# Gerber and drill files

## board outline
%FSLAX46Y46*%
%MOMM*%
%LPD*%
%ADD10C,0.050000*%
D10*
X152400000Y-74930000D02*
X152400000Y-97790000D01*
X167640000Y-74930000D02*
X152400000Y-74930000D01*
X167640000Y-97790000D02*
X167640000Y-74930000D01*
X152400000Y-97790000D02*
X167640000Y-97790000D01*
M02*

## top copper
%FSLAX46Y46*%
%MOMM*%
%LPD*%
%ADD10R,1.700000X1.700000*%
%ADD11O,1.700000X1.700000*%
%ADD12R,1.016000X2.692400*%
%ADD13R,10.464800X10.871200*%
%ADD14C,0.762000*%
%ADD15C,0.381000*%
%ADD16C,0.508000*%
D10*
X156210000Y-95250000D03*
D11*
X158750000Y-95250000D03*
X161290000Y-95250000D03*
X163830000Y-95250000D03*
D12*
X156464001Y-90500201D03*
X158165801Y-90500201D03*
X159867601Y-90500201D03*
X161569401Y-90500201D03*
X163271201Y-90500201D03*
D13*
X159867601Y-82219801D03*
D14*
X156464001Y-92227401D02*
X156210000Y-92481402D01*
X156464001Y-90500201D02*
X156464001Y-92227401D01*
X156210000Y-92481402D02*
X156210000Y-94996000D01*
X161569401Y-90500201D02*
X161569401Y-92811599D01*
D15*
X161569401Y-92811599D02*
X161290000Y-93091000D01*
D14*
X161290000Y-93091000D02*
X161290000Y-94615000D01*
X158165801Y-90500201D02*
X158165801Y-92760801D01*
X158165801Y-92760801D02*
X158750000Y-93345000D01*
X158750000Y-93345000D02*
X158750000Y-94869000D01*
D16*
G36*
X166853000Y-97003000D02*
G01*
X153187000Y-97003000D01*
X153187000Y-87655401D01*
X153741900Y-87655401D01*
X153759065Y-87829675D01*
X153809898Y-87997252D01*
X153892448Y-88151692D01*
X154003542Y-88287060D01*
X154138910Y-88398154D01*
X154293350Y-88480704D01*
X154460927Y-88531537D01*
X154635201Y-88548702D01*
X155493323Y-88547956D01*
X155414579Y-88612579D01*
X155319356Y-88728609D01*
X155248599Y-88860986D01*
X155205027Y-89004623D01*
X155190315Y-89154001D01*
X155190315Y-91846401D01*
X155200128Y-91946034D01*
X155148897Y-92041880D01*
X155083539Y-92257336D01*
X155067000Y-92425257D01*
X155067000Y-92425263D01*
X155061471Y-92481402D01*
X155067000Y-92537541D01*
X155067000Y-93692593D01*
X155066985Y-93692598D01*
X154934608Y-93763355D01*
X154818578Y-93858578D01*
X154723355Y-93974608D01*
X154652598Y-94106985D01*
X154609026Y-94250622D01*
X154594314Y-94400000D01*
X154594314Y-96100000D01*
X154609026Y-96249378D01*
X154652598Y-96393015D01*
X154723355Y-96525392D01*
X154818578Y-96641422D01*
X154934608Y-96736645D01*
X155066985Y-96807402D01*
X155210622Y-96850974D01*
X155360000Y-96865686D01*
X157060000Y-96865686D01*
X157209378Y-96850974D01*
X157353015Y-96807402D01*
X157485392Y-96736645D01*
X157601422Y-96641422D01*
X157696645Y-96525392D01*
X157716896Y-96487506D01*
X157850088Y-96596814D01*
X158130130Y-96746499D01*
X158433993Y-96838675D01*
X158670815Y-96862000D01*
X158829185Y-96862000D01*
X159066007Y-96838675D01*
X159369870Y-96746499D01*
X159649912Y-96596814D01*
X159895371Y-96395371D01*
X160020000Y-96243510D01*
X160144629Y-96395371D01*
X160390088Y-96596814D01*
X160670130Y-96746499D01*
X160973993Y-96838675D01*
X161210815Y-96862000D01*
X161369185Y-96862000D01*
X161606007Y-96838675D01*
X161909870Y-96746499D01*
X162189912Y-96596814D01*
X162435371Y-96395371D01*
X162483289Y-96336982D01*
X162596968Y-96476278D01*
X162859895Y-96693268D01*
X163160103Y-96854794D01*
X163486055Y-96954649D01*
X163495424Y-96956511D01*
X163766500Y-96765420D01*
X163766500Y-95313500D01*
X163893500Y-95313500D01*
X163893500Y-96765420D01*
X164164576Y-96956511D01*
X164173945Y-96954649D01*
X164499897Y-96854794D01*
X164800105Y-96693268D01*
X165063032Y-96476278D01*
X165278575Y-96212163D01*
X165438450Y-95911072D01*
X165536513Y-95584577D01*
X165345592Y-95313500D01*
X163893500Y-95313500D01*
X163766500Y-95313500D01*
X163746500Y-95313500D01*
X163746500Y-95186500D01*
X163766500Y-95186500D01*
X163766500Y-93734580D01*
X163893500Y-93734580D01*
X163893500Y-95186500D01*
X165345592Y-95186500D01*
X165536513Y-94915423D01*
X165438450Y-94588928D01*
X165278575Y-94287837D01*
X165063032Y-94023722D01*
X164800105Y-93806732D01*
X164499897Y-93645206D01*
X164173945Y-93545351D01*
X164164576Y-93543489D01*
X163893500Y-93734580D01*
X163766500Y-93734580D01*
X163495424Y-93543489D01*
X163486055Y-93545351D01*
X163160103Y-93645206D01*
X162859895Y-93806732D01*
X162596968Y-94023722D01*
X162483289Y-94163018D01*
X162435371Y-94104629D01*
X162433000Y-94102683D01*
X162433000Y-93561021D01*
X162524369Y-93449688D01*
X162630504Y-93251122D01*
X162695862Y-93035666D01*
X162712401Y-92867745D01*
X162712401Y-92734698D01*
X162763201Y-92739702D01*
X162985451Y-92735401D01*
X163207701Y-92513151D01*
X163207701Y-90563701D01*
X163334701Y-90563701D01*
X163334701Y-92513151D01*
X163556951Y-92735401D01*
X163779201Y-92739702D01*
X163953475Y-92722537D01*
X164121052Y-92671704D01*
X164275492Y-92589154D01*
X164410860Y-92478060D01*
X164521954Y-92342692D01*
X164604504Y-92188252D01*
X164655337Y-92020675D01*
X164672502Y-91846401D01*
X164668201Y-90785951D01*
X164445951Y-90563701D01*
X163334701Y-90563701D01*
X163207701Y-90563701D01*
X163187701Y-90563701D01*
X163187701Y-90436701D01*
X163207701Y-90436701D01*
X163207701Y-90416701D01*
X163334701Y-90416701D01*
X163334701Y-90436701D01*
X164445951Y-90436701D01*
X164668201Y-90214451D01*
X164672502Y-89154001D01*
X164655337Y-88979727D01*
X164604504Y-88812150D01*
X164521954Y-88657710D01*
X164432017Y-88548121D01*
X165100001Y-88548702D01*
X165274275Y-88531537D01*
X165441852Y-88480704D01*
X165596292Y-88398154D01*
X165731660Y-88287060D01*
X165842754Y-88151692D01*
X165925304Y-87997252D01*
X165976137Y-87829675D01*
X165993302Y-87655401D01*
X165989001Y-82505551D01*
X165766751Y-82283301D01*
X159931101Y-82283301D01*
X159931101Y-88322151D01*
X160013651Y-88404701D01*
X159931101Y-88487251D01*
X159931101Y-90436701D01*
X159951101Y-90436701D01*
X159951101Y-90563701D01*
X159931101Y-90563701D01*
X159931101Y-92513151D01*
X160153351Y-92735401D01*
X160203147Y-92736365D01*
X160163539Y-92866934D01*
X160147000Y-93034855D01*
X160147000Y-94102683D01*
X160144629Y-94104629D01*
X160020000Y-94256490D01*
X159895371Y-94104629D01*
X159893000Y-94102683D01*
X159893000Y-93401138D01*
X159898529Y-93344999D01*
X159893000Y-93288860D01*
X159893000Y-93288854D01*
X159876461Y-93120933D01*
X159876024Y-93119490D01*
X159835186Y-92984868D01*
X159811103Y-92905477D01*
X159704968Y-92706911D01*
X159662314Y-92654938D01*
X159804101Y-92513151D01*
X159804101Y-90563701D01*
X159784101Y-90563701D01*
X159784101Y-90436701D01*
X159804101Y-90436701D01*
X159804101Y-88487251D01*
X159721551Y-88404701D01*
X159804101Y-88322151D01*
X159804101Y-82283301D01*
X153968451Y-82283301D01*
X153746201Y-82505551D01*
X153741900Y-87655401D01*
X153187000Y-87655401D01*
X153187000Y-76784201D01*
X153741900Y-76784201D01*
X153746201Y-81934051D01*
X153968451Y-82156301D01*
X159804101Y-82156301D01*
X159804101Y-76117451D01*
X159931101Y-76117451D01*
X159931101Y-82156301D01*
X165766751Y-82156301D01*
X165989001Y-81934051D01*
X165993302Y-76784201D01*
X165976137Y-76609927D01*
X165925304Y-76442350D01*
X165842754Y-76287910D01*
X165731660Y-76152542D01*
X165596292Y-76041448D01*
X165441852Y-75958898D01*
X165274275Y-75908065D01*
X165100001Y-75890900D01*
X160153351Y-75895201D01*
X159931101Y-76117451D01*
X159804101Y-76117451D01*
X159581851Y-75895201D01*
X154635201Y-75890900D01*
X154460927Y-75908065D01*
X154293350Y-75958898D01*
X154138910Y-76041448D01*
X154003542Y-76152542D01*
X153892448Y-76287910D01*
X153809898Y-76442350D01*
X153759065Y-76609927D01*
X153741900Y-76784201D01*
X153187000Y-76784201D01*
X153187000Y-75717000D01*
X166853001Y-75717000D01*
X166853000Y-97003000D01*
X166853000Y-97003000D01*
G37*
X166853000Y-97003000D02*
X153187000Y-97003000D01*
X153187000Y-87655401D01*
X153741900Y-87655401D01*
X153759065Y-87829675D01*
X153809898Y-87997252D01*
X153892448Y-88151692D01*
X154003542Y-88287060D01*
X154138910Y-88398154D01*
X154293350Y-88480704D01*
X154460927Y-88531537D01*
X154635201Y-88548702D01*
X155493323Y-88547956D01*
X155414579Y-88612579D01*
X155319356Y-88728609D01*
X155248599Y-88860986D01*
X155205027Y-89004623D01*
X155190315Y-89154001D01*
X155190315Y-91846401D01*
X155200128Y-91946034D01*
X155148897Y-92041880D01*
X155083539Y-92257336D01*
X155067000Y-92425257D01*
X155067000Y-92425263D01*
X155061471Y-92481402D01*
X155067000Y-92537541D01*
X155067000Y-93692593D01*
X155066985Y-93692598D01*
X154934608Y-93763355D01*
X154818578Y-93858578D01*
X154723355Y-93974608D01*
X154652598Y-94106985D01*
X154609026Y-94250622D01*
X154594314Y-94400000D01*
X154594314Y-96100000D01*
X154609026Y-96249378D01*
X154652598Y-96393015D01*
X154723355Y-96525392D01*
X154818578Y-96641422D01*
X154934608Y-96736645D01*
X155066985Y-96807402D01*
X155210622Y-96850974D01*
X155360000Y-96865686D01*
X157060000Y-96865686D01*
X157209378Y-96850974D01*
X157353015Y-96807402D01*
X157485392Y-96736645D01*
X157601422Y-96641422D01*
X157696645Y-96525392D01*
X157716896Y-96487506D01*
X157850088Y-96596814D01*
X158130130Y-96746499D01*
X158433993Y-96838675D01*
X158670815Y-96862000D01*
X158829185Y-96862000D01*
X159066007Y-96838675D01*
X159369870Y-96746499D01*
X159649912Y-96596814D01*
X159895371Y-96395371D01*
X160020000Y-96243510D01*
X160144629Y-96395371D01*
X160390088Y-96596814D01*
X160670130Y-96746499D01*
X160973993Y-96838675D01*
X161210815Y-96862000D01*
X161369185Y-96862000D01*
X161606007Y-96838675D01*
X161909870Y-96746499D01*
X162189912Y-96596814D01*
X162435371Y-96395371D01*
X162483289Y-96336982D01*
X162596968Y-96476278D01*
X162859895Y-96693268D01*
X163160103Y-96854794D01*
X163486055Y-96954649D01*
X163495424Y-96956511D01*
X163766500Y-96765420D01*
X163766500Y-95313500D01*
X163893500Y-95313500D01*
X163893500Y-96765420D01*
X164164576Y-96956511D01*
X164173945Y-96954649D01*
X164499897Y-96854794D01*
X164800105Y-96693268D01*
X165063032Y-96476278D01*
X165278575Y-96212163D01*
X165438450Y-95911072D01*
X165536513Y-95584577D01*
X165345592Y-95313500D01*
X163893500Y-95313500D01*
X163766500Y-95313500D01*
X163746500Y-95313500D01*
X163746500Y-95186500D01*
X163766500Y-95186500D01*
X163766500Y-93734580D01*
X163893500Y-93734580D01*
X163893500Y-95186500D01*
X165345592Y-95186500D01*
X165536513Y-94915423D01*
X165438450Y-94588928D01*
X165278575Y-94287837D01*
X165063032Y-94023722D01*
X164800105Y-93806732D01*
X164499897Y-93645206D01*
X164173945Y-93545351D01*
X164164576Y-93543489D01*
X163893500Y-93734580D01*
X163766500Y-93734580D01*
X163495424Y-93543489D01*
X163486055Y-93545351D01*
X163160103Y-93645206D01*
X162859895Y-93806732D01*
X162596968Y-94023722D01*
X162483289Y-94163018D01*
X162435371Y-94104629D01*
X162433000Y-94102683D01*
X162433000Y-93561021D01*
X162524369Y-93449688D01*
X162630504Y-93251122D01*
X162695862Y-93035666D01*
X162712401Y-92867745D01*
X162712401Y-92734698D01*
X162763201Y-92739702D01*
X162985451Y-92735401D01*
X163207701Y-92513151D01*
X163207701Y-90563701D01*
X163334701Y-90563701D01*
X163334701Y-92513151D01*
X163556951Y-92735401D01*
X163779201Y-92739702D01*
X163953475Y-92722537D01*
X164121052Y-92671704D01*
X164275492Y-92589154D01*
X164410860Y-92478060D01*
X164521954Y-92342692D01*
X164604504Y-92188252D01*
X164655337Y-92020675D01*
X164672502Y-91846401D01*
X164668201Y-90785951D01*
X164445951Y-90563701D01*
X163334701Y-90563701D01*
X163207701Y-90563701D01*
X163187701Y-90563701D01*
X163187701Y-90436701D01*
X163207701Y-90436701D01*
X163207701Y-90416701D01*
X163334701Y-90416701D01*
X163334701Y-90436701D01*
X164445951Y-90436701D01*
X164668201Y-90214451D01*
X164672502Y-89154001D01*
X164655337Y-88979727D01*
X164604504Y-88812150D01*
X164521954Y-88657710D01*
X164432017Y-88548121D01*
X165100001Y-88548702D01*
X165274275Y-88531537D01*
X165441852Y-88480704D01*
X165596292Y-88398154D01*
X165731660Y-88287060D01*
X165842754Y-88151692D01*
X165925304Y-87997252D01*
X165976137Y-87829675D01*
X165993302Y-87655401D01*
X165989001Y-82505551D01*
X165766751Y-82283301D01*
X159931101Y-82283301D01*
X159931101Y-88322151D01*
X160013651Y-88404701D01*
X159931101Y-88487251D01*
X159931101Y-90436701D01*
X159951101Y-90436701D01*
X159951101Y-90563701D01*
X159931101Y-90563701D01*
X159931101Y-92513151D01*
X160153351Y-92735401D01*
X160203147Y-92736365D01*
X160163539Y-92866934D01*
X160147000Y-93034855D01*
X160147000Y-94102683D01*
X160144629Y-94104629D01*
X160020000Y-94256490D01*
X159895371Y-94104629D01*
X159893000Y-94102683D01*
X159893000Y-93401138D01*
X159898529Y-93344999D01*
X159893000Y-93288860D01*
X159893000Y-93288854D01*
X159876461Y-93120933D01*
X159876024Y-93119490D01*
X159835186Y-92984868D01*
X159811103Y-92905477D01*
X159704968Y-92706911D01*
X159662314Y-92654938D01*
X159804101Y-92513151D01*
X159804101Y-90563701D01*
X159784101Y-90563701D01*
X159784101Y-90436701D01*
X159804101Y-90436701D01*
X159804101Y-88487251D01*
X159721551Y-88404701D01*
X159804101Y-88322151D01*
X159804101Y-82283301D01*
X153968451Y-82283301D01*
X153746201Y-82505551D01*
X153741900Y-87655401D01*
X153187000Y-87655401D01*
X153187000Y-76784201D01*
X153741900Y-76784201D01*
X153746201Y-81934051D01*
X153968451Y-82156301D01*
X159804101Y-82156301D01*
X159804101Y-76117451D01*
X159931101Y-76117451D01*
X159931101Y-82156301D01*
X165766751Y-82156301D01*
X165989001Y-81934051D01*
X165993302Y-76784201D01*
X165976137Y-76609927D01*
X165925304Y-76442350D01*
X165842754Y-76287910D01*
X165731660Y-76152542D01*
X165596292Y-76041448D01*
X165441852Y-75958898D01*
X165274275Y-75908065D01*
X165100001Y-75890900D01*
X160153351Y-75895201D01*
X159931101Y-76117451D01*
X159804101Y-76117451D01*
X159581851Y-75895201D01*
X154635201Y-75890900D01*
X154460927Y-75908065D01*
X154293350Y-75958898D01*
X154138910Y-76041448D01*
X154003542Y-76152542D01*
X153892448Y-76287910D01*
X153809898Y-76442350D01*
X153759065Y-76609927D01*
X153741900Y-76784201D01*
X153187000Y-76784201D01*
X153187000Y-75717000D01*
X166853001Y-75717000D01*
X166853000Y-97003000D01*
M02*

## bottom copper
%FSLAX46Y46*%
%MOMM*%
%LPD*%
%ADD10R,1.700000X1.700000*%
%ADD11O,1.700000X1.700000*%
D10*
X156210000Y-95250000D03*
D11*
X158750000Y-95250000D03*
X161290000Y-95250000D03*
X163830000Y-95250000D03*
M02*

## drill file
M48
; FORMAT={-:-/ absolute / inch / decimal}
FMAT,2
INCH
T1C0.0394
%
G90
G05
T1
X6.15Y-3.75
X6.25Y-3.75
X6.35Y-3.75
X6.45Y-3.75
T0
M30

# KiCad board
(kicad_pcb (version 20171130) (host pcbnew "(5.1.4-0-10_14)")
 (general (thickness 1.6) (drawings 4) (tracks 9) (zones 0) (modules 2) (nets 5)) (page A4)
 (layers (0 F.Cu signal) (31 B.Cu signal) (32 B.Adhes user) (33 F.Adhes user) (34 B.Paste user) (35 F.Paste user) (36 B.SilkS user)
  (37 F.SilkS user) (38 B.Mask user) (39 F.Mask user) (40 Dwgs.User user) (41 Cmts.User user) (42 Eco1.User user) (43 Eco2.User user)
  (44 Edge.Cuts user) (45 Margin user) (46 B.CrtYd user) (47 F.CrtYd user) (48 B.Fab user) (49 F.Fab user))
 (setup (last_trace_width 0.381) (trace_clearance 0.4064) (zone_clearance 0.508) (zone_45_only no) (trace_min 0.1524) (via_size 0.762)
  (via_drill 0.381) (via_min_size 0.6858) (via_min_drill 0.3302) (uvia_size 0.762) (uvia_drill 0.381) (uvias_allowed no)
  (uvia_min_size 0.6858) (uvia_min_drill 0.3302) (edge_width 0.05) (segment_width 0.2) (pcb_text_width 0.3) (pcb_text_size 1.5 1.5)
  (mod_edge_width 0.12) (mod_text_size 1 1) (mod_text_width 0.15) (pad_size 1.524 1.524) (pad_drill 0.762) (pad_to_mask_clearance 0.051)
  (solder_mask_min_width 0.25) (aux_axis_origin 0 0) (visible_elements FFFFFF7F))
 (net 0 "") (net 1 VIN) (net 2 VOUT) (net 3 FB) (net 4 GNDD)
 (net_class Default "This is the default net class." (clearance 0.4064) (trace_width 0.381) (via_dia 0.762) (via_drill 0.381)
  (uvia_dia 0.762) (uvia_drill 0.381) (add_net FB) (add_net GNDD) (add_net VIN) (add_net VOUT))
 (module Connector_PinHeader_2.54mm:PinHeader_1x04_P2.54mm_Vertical (layer F.Cu) (at 156.21 95.25 90)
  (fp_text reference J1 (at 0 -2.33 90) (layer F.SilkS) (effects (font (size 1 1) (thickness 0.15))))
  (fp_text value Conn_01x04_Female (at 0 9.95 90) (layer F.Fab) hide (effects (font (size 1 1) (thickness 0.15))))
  (pad 1 thru_hole rect (at 0 0 90) (size 1.7 1.7) (drill 1) (layers *.Cu *.Mask) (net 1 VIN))
  (pad 2 thru_hole oval (at 0 2.54 90) (size 1.7 1.7) (drill 1) (layers *.Cu *.Mask) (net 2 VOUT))
  (pad 3 thru_hole oval (at 0 5.08 90) (size 1.7 1.7) (drill 1) (layers *.Cu *.Mask) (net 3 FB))
  (pad 4 thru_hole oval (at 0 7.62 90) (size 1.7 1.7) (drill 1) (layers *.Cu *.Mask) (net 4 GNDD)))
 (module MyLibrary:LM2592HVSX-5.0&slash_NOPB (layer F.Cu) (at 159.867601 82.219801)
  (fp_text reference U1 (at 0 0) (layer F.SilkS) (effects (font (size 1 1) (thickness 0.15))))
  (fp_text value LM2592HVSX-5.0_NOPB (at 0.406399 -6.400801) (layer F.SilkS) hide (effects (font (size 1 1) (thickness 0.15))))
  (pad 1 smd rect (at -3.4036 8.2804) (size 1.016 2.6924) (layers F.Cu F.Paste F.Mask) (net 1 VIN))
  (pad 2 smd rect (at -1.7018 8.2804) (size 1.016 2.6924) (layers F.Cu F.Paste F.Mask) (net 2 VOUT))
  (pad 3 smd rect (at 0 8.2804) (size 1.016 2.6924) (layers F.Cu F.Paste F.Mask) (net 4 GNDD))
  (pad 4 smd rect (at 1.7018 8.2804) (size 1.016 2.6924) (layers F.Cu F.Paste F.Mask) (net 3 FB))
  (pad 5 smd rect (at 3.4036 8.2804) (size 1.016 2.6924) (layers F.Cu F.Paste F.Mask) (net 4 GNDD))
  (pad 6 smd rect (at 0 0) (size 10.4648 10.8712) (layers F.Cu F.Paste F.Mask) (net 4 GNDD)))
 (gr_line (start 152.4 74.93) (end 152.4 97.79) (layer Edge.Cuts) (width 0.05))
 (gr_line (start 167.64 74.93) (end 152.4 74.93) (layer Edge.Cuts) (width 0.05))
 (gr_line (start 167.64 97.79) (end 167.64 74.93) (layer Edge.Cuts) (width 0.05))
 (gr_line (start 152.4 97.79) (end 167.64 97.79) (layer Edge.Cuts) (width 0.05))
 (segment (start 156.464001 92.227401) (end 156.21 92.481402) (width 0.762) (layer F.Cu) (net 1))
 (segment (start 156.464001 90.500201) (end 156.464001 92.227401) (width 0.762) (layer F.Cu) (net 1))
 (segment (start 156.21 92.481402) (end 156.21 94.996) (width 0.762) (layer F.Cu) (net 1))
 (segment (start 161.569401 90.500201) (end 161.569401 92.811599) (width 0.762) (layer F.Cu) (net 3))
 (segment (start 161.569401 92.811599) (end 161.29 93.091) (width 0.381) (layer F.Cu) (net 3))
 (segment (start 161.29 93.091) (end 161.29 94.615) (width 0.762) (layer F.Cu) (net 3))
 (segment (start 158.165801 90.500201) (end 158.165801 92.760801) (width 0.762) (layer F.Cu) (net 2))
 (segment (start 158.165801 92.760801) (end 158.75 93.345) (width 0.762) (layer F.Cu) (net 2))
 (segment (start 158.75 93.345) (end 158.75 94.869) (width 0.762) (layer F.Cu) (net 2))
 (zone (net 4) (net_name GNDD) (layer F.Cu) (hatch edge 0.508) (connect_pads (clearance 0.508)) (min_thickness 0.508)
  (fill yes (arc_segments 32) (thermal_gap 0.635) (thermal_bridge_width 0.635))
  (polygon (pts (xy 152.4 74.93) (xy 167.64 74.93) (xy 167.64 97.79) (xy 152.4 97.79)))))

